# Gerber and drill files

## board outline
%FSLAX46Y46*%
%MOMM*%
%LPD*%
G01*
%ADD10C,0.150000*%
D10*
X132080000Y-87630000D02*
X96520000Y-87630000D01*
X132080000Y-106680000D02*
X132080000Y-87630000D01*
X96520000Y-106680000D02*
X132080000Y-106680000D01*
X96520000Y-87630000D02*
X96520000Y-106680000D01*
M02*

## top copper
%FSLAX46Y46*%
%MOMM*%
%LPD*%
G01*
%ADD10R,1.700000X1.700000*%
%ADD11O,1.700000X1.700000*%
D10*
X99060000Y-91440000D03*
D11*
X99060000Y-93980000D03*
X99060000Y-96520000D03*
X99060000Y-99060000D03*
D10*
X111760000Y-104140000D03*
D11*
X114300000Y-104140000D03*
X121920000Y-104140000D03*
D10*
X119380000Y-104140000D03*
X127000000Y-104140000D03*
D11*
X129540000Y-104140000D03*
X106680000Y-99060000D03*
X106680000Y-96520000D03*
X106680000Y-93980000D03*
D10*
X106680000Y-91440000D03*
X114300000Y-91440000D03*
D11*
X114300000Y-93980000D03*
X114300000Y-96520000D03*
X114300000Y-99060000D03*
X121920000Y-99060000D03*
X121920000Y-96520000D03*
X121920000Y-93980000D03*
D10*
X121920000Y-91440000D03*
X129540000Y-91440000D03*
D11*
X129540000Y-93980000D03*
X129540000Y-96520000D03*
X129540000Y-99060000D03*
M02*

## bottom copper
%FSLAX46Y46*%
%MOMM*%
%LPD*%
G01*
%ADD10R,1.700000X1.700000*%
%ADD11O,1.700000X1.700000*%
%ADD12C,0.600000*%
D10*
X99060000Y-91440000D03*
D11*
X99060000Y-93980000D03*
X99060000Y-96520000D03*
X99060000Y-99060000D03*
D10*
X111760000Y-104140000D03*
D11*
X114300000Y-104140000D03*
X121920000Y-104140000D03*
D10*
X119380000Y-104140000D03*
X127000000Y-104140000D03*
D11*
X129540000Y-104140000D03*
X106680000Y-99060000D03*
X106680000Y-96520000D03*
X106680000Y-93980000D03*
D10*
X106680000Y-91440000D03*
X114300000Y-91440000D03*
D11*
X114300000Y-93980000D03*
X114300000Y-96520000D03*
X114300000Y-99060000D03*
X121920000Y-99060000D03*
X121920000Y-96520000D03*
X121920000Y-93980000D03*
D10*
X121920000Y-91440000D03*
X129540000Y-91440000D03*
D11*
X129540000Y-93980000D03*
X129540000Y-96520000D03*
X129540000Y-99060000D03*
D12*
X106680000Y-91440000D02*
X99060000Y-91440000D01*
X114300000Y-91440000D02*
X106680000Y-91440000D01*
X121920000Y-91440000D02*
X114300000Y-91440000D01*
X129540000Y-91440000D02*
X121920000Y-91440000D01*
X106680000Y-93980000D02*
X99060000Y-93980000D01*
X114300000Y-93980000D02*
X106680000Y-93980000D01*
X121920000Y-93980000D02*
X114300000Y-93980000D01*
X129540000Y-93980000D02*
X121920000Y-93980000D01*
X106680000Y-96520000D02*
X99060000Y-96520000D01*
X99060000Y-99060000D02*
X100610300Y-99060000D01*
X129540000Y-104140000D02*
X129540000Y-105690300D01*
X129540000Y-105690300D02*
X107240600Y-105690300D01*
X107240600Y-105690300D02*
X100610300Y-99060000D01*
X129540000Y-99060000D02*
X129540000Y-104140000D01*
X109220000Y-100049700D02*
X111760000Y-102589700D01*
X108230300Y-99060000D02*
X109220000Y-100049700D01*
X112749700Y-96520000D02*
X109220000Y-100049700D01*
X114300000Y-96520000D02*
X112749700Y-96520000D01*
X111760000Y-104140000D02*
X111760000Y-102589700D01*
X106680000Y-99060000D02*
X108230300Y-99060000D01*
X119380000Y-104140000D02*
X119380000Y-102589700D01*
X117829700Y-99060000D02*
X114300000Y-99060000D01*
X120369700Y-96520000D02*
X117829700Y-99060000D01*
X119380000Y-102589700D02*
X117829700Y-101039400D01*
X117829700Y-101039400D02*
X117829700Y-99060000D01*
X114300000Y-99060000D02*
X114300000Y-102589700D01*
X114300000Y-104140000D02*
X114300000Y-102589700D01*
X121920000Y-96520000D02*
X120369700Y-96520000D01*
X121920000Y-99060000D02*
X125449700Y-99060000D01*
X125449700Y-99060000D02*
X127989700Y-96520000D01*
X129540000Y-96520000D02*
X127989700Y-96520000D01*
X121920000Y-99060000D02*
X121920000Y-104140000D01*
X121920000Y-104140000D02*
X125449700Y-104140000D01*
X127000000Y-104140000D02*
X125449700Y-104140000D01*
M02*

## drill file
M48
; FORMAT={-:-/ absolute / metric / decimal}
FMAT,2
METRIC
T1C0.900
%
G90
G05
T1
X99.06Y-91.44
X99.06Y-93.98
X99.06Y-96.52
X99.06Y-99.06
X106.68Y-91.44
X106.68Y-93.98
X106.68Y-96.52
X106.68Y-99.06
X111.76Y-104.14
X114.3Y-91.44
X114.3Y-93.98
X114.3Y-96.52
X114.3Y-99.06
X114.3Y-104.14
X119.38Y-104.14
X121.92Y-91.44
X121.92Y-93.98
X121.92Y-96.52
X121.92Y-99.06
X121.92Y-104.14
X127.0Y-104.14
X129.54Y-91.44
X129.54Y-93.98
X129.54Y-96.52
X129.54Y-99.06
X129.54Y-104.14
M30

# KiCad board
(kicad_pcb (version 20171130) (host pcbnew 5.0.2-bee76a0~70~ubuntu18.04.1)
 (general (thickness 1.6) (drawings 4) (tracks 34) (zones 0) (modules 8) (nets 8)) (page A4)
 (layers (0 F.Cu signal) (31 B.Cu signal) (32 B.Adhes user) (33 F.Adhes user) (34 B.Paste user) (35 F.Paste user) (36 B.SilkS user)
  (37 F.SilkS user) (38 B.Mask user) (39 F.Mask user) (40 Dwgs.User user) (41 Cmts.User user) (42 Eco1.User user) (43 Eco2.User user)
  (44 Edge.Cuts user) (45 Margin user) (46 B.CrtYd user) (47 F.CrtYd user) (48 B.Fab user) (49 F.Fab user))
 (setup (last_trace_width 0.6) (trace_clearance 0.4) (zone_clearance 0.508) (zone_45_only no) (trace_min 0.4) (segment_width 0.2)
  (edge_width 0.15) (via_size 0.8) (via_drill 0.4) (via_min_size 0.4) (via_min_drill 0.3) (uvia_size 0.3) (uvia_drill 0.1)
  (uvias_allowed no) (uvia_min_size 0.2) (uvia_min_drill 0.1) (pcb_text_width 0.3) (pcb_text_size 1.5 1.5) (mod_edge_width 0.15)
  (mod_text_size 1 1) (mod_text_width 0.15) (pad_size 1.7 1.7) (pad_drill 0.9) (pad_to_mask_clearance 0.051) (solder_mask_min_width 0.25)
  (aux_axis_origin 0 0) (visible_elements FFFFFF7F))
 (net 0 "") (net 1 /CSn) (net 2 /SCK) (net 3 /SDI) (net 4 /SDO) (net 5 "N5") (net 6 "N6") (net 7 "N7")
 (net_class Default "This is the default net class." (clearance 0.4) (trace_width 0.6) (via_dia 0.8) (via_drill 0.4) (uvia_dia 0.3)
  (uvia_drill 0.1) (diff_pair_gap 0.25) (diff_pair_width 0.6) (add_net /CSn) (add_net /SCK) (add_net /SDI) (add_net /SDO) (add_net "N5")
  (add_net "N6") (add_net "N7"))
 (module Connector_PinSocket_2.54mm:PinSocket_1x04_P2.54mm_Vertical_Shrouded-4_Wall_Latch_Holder (layer F.Cu) (at 99.06 91.44)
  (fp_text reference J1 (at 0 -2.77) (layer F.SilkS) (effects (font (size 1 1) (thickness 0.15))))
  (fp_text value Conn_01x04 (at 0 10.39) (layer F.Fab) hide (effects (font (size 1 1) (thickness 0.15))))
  (pad 1 thru_hole rect (at 0 0) (size 1.7 1.7) (drill 0.9) (layers *.Cu *.Mask) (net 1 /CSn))
  (pad 2 thru_hole oval (at 0 2.54) (size 1.7 1.7) (drill 0.9) (layers *.Cu *.Mask) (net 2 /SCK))
  (pad 3 thru_hole oval (at 0 5.08) (size 1.7 1.7) (drill 0.9) (layers *.Cu *.Mask) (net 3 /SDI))
  (pad 4 thru_hole oval (at 0 7.62) (size 1.7 1.7) (drill 0.9) (layers *.Cu *.Mask) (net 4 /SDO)))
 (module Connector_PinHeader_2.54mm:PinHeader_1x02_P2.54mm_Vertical (layer F.Cu) (at 111.76 104.14 90)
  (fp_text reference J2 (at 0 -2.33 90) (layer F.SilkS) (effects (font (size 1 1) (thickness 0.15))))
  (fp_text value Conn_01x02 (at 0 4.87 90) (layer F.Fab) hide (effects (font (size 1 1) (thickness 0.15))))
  (pad 1 thru_hole rect (at 0 0 90) (size 1.7 1.7) (drill 0.9) (layers *.Cu *.Mask) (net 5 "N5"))
  (pad 2 thru_hole oval (at 0 2.54 90) (size 1.7 1.7) (drill 0.9) (layers *.Cu *.Mask) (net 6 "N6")))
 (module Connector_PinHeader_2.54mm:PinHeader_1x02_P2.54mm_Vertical (layer F.Cu) (at 119.38 104.14 90)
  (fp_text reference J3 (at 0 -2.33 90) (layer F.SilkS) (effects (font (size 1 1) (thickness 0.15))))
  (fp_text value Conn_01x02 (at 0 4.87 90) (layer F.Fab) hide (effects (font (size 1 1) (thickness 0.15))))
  (pad 2 thru_hole oval (at 0 2.54 90) (size 1.7 1.7) (drill 0.9) (layers *.Cu *.Mask) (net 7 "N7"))
  (pad 1 thru_hole rect (at 0 0 90) (size 1.7 1.7) (drill 0.9) (layers *.Cu *.Mask) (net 6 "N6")))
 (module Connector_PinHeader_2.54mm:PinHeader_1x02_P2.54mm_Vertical (layer F.Cu) (at 127 104.14 90)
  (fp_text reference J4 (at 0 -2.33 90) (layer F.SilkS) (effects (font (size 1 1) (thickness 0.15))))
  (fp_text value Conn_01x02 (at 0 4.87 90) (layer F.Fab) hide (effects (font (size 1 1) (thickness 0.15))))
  (pad 1 thru_hole rect (at 0 0 90) (size 1.7 1.7) (drill 0.9) (layers *.Cu *.Mask) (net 7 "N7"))
  (pad 2 thru_hole oval (at 0 2.54 90) (size 1.7 1.7) (drill 0.9) (layers *.Cu *.Mask) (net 4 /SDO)))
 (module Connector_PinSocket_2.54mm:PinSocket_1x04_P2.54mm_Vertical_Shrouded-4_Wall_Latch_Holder (layer F.Cu) (at 106.68 91.44)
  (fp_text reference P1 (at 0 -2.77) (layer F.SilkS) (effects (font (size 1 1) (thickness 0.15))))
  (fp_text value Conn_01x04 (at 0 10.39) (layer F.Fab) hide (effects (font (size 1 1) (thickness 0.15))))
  (pad 4 thru_hole oval (at 0 7.62) (size 1.7 1.7) (drill 0.9) (layers *.Cu *.Mask) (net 5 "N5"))
  (pad 3 thru_hole oval (at 0 5.08) (size 1.7 1.7) (drill 0.9) (layers *.Cu *.Mask) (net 3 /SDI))
  (pad 2 thru_hole oval (at 0 2.54) (size 1.7 1.7) (drill 0.9) (layers *.Cu *.Mask) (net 2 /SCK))
  (pad 1 thru_hole rect (at 0 0) (size 1.7 1.7) (drill 0.9) (layers *.Cu *.Mask) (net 1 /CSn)))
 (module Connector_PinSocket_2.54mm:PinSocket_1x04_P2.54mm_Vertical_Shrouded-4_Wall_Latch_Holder (layer F.Cu) (at 114.3 91.44)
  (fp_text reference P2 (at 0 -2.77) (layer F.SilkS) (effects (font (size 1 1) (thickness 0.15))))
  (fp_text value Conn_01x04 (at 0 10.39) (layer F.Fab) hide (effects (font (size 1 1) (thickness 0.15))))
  (pad 1 thru_hole rect (at 0 0) (size 1.7 1.7) (drill 0.9) (layers *.Cu *.Mask) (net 1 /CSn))
  (pad 2 thru_hole oval (at 0 2.54) (size 1.7 1.7) (drill 0.9) (layers *.Cu *.Mask) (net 2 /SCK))
  (pad 3 thru_hole oval (at 0 5.08) (size 1.7 1.7) (drill 0.9) (layers *.Cu *.Mask) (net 5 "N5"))
  (pad 4 thru_hole oval (at 0 7.62) (size 1.7 1.7) (drill 0.9) (layers *.Cu *.Mask) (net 6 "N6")))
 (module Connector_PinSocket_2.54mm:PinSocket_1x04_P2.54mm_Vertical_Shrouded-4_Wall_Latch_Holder (layer F.Cu) (at 121.92 91.44)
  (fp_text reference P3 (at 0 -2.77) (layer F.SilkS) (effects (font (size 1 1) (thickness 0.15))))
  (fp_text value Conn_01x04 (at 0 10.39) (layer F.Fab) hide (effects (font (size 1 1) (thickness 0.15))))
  (pad 4 thru_hole oval (at 0 7.62) (size 1.7 1.7) (drill 0.9) (layers *.Cu *.Mask) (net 7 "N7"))
  (pad 3 thru_hole oval (at 0 5.08) (size 1.7 1.7) (drill 0.9) (layers *.Cu *.Mask) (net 6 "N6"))
  (pad 2 thru_hole oval (at 0 2.54) (size 1.7 1.7) (drill 0.9) (layers *.Cu *.Mask) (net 2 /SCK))
  (pad 1 thru_hole rect (at 0 0) (size 1.7 1.7) (drill 0.9) (layers *.Cu *.Mask) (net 1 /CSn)))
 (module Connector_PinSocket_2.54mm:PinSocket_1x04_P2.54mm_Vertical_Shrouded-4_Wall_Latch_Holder (layer F.Cu) (at 129.54 91.44)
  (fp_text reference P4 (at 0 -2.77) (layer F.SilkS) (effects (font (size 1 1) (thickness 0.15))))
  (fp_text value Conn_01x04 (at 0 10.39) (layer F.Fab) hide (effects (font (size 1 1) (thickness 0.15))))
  (pad 1 thru_hole rect (at 0 0) (size 1.7 1.7) (drill 0.9) (layers *.Cu *.Mask) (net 1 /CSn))
  (pad 2 thru_hole oval (at 0 2.54) (size 1.7 1.7) (drill 0.9) (layers *.Cu *.Mask) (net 2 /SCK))
  (pad 3 thru_hole oval (at 0 5.08) (size 1.7 1.7) (drill 0.9) (layers *.Cu *.Mask) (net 7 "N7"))
  (pad 4 thru_hole oval (at 0 7.62) (size 1.7 1.7) (drill 0.9) (layers *.Cu *.Mask) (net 4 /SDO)))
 (gr_line (start 132.08 87.63) (end 96.52 87.63) (layer Edge.Cuts) (width 0.15))
 (gr_line (start 132.08 106.68) (end 132.08 87.63) (layer Edge.Cuts) (width 0.15))
 (gr_line (start 96.52 106.68) (end 132.08 106.68) (layer Edge.Cuts) (width 0.15))
 (gr_line (start 96.52 87.63) (end 96.52 106.68) (layer Edge.Cuts) (width 0.15))
 (segment (start 106.68 91.44) (end 99.06 91.44) (width 0.6) (layer B.Cu) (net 1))
 (segment (start 114.3 91.44) (end 106.68 91.44) (width 0.6) (layer B.Cu) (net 1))
 (segment (start 121.92 91.44) (end 114.3 91.44) (width 0.6) (layer B.Cu) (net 1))
 (segment (start 129.54 91.44) (end 121.92 91.44) (width 0.6) (layer B.Cu) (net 1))
 (segment (start 106.68 93.98) (end 99.06 93.98) (width 0.6) (layer B.Cu) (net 2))
 (segment (start 114.3 93.98) (end 106.68 93.98) (width 0.6) (layer B.Cu) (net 2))
 (segment (start 121.92 93.98) (end 114.3 93.98) (width 0.6) (layer B.Cu) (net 2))
 (segment (start 129.54 93.98) (end 121.92 93.98) (width 0.6) (layer B.Cu) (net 2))
 (segment (start 106.68 96.52) (end 99.06 96.52) (width 0.6) (layer B.Cu) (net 3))
 (segment (start 99.06 99.06) (end 100.6103 99.06) (width 0.6) (layer B.Cu) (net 4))
 (segment (start 129.54 104.14) (end 129.54 105.6903) (width 0.6) (layer B.Cu) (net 4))
 (segment (start 129.54 105.6903) (end 107.2406 105.6903) (width 0.6) (layer B.Cu) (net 4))
 (segment (start 107.2406 105.6903) (end 100.6103 99.06) (width 0.6) (layer B.Cu) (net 4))
 (segment (start 129.54 99.06) (end 129.54 104.14) (width 0.6) (layer B.Cu) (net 4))
 (segment (start 109.22 100.0497) (end 111.76 102.5897) (width 0.6) (layer B.Cu) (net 5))
 (segment (start 108.2303 99.06) (end 109.22 100.0497) (width 0.6) (layer B.Cu) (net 5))
 (segment (start 112.7497 96.52) (end 109.22 100.0497) (width 0.6) (layer B.Cu) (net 5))
 (segment (start 114.3 96.52) (end 112.7497 96.52) (width 0.6) (layer B.Cu) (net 5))
 (segment (start 111.76 104.14) (end 111.76 102.5897) (width 0.6) (layer B.Cu) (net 5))
 (segment (start 106.68 99.06) (end 108.2303 99.06) (width 0.6) (layer B.Cu) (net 5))
 (segment (start 119.38 104.14) (end 119.38 102.5897) (width 0.6) (layer B.Cu) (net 6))
 (segment (start 117.8297 99.06) (end 114.3 99.06) (width 0.6) (layer B.Cu) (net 6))
 (segment (start 120.3697 96.52) (end 117.8297 99.06) (width 0.6) (layer B.Cu) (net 6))
 (segment (start 119.38 102.5897) (end 117.8297 101.0394) (width 0.6) (layer B.Cu) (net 6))
 (segment (start 117.8297 101.0394) (end 117.8297 99.06) (width 0.6) (layer B.Cu) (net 6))
 (segment (start 114.3 99.06) (end 114.3 102.5897) (width 0.6) (layer B.Cu) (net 6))
 (segment (start 114.3 104.14) (end 114.3 102.5897) (width 0.6) (layer B.Cu) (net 6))
 (segment (start 121.92 96.52) (end 120.3697 96.52) (width 0.6) (layer B.Cu) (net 6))
 (segment (start 121.92 99.06) (end 125.4497 99.06) (width 0.6) (layer B.Cu) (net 7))
 (segment (start 125.4497 99.06) (end 127.9897 96.52) (width 0.6) (layer B.Cu) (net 7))
 (segment (start 129.54 96.52) (end 127.9897 96.52) (width 0.6) (layer B.Cu) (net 7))
 (segment (start 121.92 99.06) (end 121.92 104.14) (width 0.6) (layer B.Cu) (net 7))
 (segment (start 121.92 104.14) (end 125.4497 104.14) (width 0.6) (layer B.Cu) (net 7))
 (segment (start 127 104.14) (end 125.4497 104.14) (width 0.6) (layer B.Cu) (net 7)))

